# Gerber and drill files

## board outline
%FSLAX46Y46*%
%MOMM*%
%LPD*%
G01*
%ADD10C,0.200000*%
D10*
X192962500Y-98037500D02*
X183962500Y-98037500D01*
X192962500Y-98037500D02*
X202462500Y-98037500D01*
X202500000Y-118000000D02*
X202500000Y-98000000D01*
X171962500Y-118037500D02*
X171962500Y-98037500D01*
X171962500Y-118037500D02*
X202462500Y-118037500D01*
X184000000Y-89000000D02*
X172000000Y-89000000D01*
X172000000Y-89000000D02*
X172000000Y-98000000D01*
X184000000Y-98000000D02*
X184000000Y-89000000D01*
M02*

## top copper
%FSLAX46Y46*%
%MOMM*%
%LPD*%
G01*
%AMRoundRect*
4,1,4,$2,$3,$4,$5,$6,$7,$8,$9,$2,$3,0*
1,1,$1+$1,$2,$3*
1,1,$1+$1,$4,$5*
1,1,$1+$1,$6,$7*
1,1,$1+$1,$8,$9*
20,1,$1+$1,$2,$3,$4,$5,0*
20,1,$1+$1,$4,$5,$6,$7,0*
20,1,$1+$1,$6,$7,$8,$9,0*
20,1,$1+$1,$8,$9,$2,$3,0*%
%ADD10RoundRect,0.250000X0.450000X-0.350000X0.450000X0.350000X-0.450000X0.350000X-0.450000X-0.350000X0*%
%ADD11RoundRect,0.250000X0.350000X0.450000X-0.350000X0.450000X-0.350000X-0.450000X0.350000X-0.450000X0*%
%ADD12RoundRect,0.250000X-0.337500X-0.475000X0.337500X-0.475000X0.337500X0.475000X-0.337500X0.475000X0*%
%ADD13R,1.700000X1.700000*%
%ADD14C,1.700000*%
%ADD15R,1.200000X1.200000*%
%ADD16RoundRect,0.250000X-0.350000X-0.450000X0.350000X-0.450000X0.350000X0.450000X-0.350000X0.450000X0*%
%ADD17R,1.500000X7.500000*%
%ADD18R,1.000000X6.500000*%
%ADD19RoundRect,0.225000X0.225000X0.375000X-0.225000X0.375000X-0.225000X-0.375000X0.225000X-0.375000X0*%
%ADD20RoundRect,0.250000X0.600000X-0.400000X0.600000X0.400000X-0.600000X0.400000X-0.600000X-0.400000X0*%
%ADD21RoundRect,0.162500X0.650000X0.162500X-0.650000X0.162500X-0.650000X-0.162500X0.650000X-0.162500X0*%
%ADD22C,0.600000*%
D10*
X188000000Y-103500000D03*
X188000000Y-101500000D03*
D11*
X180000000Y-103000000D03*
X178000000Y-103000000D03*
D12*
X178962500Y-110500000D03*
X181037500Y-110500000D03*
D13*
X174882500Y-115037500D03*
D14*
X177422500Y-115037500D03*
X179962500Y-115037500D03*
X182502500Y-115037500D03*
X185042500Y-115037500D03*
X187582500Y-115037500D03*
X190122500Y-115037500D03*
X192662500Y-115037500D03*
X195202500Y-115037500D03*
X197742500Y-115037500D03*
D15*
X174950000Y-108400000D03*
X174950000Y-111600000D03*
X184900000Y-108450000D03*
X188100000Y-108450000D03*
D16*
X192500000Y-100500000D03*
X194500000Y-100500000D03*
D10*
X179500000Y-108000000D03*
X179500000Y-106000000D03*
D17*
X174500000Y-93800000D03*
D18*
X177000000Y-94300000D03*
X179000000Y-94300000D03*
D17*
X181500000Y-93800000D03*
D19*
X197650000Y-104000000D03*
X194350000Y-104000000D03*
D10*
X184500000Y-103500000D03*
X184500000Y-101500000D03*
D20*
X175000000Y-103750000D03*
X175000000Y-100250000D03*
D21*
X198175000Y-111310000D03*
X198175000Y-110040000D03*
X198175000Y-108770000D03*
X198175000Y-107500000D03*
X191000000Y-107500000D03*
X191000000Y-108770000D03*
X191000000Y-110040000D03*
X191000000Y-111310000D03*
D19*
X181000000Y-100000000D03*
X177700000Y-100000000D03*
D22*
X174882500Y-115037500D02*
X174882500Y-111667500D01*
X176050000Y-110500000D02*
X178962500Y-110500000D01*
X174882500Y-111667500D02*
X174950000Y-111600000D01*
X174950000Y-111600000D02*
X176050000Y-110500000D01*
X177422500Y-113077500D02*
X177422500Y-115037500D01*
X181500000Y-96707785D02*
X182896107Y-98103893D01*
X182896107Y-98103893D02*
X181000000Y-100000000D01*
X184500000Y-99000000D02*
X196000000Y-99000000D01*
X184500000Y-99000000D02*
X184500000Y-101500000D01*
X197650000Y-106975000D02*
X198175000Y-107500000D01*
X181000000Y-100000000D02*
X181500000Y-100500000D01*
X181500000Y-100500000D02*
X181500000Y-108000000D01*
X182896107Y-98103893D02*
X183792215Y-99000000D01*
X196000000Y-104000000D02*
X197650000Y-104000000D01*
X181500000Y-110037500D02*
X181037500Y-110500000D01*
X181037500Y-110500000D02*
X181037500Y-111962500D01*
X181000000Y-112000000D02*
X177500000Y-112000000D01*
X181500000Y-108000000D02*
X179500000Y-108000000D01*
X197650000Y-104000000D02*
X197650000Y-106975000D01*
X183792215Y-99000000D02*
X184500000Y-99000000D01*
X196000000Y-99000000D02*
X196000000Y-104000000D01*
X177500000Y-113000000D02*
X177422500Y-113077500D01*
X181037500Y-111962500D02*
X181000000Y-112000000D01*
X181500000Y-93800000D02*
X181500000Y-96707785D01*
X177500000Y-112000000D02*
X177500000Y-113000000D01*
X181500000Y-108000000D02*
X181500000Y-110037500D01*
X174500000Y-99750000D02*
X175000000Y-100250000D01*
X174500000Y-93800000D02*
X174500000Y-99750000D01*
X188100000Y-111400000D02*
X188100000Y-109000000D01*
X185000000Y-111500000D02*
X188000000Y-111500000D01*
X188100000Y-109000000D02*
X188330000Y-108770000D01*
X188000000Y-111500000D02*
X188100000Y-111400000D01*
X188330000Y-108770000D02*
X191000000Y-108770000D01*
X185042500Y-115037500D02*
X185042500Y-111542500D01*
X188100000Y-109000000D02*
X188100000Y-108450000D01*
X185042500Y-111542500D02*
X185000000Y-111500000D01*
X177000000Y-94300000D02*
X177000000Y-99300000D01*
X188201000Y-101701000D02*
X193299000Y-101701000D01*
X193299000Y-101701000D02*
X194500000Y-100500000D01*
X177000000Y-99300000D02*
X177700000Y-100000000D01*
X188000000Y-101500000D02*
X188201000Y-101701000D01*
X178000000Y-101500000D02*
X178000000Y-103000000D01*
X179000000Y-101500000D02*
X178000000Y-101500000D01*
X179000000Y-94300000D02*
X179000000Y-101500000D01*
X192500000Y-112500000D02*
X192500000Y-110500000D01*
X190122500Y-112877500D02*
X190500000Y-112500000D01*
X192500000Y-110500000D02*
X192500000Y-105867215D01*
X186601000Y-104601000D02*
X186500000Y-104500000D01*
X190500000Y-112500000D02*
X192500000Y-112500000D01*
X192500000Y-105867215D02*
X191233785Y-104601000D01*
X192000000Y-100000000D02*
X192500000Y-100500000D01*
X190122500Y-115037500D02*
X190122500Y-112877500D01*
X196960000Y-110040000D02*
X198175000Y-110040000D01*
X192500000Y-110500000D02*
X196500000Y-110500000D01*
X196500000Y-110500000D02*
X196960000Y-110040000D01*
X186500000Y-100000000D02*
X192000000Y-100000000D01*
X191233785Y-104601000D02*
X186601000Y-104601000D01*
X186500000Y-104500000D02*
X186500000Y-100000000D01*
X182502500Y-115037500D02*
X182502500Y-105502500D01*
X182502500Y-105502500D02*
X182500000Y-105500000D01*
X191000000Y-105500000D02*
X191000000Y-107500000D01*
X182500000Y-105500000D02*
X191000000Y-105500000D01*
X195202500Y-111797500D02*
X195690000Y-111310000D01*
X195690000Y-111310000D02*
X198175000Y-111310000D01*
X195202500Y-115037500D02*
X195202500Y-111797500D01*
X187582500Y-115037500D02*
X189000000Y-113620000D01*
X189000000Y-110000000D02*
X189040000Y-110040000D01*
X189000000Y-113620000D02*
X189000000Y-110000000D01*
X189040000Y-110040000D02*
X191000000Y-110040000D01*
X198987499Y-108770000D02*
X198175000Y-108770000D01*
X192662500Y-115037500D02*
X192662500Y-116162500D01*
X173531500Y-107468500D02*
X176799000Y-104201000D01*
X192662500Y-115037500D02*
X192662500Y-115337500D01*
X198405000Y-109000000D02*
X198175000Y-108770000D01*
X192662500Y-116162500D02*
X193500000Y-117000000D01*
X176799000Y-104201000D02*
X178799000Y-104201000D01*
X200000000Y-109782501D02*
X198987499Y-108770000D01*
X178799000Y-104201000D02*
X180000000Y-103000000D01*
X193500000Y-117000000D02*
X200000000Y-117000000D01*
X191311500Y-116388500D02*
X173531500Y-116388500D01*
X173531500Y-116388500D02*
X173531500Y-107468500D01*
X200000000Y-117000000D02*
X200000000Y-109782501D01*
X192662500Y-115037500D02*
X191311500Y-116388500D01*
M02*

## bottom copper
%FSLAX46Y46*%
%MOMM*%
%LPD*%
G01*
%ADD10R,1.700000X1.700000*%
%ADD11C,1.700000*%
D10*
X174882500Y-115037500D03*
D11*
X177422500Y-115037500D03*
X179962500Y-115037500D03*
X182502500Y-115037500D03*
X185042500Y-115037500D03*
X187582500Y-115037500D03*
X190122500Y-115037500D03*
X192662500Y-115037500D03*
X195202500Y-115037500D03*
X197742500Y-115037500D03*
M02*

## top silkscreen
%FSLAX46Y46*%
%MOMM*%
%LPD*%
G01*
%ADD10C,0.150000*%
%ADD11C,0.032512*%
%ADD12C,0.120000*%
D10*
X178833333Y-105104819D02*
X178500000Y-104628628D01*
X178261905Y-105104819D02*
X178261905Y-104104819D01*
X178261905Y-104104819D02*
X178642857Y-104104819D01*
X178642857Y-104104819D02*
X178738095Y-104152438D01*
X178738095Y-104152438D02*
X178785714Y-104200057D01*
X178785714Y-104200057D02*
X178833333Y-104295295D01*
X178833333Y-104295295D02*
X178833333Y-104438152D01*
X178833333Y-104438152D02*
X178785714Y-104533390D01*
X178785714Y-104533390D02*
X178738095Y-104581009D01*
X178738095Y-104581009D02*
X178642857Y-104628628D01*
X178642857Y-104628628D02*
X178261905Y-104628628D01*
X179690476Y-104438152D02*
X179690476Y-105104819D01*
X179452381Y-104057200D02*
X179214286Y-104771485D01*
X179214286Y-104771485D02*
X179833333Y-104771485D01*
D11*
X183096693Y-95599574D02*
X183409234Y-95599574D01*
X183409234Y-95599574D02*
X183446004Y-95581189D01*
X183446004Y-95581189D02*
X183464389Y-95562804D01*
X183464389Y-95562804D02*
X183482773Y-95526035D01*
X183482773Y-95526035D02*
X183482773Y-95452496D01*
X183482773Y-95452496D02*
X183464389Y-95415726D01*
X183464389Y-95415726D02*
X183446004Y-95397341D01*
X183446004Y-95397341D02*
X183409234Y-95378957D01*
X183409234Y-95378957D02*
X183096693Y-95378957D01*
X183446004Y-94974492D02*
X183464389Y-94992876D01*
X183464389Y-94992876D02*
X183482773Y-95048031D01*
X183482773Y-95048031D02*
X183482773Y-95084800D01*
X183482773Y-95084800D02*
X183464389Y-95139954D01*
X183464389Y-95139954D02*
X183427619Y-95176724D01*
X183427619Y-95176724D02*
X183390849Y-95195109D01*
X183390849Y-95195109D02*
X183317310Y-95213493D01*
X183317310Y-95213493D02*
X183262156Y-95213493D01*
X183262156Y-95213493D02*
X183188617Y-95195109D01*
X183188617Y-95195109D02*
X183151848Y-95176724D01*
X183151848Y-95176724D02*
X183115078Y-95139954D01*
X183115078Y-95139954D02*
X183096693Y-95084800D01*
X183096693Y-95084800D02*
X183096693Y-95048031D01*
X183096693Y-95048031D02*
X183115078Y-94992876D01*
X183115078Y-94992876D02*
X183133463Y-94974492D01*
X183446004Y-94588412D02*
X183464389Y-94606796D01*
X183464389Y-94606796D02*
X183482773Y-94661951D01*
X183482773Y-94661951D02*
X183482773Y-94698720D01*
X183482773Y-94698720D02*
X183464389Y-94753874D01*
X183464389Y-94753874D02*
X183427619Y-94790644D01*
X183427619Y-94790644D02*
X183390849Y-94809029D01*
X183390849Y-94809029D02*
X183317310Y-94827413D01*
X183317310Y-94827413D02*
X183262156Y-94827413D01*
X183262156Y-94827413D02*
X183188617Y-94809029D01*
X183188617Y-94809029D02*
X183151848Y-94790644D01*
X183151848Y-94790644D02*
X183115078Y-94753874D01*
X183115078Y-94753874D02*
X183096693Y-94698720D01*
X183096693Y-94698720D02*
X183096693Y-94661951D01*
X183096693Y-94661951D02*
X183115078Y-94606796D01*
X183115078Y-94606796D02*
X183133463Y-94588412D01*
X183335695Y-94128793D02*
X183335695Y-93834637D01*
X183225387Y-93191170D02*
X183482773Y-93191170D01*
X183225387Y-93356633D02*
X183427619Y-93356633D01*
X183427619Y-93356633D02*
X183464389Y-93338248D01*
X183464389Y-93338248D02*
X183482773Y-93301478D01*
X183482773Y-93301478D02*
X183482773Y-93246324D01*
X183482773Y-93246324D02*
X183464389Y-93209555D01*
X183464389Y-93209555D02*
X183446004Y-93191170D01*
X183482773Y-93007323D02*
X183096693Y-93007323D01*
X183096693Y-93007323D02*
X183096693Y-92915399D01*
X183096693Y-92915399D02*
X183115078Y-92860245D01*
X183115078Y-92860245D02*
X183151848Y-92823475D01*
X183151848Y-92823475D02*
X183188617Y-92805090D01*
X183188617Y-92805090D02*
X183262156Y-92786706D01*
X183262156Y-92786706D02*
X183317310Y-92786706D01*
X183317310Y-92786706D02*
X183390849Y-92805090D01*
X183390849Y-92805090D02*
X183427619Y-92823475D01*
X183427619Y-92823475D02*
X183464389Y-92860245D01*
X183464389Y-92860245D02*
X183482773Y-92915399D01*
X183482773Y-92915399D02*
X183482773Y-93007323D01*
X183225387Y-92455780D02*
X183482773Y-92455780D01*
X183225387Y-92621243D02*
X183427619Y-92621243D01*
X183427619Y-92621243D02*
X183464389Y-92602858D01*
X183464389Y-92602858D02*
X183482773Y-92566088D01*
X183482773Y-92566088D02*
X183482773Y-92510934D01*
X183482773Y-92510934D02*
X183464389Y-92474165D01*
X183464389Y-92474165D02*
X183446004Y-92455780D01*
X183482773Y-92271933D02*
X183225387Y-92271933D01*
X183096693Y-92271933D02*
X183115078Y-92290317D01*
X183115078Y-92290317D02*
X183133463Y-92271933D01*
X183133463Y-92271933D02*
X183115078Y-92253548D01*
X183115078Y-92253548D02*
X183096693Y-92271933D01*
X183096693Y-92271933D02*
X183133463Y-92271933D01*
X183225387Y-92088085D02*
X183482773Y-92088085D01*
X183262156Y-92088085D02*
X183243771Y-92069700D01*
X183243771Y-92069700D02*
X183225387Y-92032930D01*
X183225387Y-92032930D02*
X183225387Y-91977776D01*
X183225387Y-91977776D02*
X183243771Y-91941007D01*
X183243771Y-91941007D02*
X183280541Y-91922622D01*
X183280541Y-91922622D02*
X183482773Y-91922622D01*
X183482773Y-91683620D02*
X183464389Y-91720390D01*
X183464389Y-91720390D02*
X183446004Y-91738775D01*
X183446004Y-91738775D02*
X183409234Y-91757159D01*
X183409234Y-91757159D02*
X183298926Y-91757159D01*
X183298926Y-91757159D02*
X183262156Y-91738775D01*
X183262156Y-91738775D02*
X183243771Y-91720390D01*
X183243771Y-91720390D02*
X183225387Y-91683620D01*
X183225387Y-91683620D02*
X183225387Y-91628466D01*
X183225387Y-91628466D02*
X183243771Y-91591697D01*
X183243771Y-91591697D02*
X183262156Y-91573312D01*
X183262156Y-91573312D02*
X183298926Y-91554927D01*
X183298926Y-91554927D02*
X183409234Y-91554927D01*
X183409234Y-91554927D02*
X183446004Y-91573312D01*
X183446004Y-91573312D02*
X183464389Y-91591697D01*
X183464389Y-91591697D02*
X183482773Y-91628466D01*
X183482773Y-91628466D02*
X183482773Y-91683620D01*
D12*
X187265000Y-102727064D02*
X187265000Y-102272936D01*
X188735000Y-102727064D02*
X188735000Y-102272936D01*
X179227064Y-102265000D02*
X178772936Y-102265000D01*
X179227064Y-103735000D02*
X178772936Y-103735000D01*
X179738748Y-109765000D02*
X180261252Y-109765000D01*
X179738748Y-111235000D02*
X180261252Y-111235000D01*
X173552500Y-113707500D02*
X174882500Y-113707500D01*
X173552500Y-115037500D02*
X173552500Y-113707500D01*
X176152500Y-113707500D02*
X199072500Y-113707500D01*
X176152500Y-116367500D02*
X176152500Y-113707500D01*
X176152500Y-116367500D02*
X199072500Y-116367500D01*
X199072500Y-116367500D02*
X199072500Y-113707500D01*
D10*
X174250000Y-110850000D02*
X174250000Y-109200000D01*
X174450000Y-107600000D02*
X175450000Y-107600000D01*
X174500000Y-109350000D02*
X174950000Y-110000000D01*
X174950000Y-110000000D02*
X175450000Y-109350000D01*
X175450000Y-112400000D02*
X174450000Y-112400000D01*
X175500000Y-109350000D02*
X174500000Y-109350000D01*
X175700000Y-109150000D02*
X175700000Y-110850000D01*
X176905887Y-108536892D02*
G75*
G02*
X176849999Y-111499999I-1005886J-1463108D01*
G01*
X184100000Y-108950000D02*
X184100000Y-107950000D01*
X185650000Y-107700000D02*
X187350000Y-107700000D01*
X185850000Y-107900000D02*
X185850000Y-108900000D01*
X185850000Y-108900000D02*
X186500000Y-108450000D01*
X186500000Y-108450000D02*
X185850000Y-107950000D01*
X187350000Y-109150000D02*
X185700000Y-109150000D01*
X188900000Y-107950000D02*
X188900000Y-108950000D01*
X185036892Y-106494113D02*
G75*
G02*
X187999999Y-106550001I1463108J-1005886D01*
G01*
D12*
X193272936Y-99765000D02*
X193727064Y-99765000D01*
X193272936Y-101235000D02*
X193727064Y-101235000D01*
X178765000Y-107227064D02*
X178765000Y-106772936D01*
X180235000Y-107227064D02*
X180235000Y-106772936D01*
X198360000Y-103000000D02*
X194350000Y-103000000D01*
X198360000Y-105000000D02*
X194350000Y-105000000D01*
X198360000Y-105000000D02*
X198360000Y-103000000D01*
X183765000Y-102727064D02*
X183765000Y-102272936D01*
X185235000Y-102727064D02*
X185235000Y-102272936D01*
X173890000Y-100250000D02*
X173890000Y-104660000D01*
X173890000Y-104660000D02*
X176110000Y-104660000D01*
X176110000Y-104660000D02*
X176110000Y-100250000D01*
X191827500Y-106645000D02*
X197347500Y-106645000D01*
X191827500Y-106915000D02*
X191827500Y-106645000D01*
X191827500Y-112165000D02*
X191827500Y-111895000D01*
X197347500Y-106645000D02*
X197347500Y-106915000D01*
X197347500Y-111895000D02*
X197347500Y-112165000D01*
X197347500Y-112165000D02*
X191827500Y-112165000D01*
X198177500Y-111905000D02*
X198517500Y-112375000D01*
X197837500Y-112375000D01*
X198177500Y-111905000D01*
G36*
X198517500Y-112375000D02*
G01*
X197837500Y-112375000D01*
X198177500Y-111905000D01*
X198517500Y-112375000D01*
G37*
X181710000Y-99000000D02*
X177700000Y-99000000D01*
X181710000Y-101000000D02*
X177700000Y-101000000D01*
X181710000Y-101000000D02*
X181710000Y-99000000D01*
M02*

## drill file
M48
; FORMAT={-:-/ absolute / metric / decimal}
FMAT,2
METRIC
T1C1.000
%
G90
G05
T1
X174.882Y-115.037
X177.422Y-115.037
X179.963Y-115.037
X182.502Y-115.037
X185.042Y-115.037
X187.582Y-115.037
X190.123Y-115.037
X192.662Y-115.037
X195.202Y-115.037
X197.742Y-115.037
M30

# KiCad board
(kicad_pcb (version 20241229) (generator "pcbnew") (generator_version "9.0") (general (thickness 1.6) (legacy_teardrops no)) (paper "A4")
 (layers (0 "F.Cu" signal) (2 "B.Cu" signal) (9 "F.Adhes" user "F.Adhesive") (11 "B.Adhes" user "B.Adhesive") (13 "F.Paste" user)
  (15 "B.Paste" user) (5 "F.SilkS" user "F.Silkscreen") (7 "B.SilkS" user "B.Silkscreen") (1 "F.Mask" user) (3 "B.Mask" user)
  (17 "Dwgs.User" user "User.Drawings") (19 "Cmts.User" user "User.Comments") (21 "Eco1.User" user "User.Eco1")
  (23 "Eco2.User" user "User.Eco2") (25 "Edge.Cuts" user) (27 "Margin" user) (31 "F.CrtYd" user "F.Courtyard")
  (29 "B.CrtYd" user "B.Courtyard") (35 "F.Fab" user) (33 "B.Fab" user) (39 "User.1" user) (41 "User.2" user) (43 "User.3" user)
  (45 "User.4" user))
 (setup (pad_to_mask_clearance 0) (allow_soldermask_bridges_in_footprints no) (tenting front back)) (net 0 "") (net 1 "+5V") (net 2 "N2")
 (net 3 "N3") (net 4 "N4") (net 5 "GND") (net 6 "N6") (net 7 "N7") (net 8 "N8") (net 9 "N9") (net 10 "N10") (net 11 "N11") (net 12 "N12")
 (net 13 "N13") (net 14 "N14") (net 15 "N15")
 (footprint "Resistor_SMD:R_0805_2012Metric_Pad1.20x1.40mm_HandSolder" (layer "F.Cu") (at 188 102.5 90)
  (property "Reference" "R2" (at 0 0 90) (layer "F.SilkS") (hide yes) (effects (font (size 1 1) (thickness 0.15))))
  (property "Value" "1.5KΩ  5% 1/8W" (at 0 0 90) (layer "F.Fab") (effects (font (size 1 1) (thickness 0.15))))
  (fp_line (start -0.227064 -0.735) (end 0.227064 -0.735) (stroke (width 0.12) (type solid)) (layer "F.SilkS"))
  (fp_line (start -0.227064 0.735) (end 0.227064 0.735) (stroke (width 0.12) (type solid)) (layer "F.SilkS"))
  (pad "1" smd roundrect (at -1 0 90) (size 1.2 1.4) (layers "F.Cu" "F.Mask" "F.Paste") (roundrect_rratio 0.208333) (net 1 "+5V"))
  (pad "2" smd roundrect (at 1 0 90) (size 1.2 1.4) (layers "F.Cu" "F.Mask" "F.Paste") (roundrect_rratio 0.208333) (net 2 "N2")))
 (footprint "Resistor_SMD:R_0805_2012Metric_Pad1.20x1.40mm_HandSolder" (layer "F.Cu") (at 179 103 180)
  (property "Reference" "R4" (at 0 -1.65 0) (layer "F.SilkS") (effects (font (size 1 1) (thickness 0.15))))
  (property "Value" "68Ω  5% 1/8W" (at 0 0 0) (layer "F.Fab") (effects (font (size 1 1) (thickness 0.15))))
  (fp_line (start -0.227064 0.735) (end 0.227064 0.735) (stroke (width 0.12) (type solid)) (layer "F.SilkS"))
  (fp_line (start -0.227064 -0.735) (end 0.227064 -0.735) (stroke (width 0.12) (type solid)) (layer "F.SilkS"))
  (pad "1" smd roundrect (at -1 0 180) (size 1.2 1.4) (layers "F.Cu" "F.Mask" "F.Paste") (roundrect_rratio 0.208333) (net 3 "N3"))
  (pad "2" smd roundrect (at 1 0 180) (size 1.2 1.4) (layers "F.Cu" "F.Mask" "F.Paste") (roundrect_rratio 0.208333) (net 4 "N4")))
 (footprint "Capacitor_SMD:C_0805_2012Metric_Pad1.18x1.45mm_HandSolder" (layer "F.Cu") (at 180 110.5)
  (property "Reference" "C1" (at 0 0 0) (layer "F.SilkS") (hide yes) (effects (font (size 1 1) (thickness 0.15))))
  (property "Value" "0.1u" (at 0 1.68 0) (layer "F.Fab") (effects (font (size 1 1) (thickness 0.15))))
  (fp_line (start -0.261252 -0.735) (end 0.261252 -0.735) (stroke (width 0.12) (type solid)) (layer "F.SilkS"))
  (fp_line (start -0.261252 0.735) (end 0.261252 0.735) (stroke (width 0.12) (type solid)) (layer "F.SilkS"))
  (pad "1" smd roundrect (at -1.0375 0) (size 1.175 1.45) (layers "F.Cu" "F.Mask" "F.Paste") (roundrect_rratio 0.212766) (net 1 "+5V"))
  (pad "2" smd roundrect (at 1.0375 0) (size 1.175 1.45) (layers "F.Cu" "F.Mask" "F.Paste") (roundrect_rratio 0.212766) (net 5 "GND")))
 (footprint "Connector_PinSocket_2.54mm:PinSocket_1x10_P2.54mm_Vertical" (layer "F.Cu") (at 174.8825 115.0375 90)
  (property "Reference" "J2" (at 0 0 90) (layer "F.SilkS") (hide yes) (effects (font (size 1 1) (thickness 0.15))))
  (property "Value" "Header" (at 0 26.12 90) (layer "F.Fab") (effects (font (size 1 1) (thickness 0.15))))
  (fp_line (start 1.33 -1.33) (end 1.33 0) (stroke (width 0.12) (type solid)) (layer "F.SilkS"))
  (fp_line (start 0 -1.33) (end 1.33 -1.33) (stroke (width 0.12) (type solid)) (layer "F.SilkS"))
  (fp_line (start 1.33 1.27) (end 1.33 24.19) (stroke (width 0.12) (type solid)) (layer "F.SilkS"))
  (fp_line (start -1.33 1.27) (end 1.33 1.27) (stroke (width 0.12) (type solid)) (layer "F.SilkS"))
  (fp_line (start -1.33 1.27) (end -1.33 24.19) (stroke (width 0.12) (type solid)) (layer "F.SilkS"))
  (fp_line (start -1.33 24.19) (end 1.33 24.19) (stroke (width 0.12) (type solid)) (layer "F.SilkS"))
  (pad "1" thru_hole rect (at 0 0 90) (size 1.7 1.7) (drill 1) (layers "*.Cu" "*.Mask") (remove_unused_layers no) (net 1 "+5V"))
  (pad "2" thru_hole circle (at 0 2.54 90) (size 1.7 1.7) (drill 1) (layers "*.Cu" "*.Mask") (remove_unused_layers no) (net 5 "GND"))
  (pad "3" thru_hole circle (at 0 5.08 90) (size 1.7 1.7) (drill 1) (layers "*.Cu" "*.Mask") (remove_unused_layers no) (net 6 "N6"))
  (pad "4" thru_hole circle (at 0 7.62 90) (size 1.7 1.7) (drill 1) (layers "*.Cu" "*.Mask") (remove_unused_layers no) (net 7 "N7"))
  (pad "5" thru_hole circle (at 0 10.16 90) (size 1.7 1.7) (drill 1) (layers "*.Cu" "*.Mask") (remove_unused_layers no) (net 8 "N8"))
  (pad "6" thru_hole circle (at 0 12.7 90) (size 1.7 1.7) (drill 1) (layers "*.Cu" "*.Mask") (remove_unused_layers no) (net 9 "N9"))
  (pad "7" thru_hole circle (at 0 15.24 90) (size 1.7 1.7) (drill 1) (layers "*.Cu" "*.Mask") (remove_unused_layers no) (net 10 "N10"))
  (pad "8" thru_hole circle (at 0 17.78 90) (size 1.7 1.7) (drill 1) (layers "*.Cu" "*.Mask") (remove_unused_layers no) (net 3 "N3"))
  (pad "9" thru_hole circle (at 0 20.32 90) (size 1.7 1.7) (drill 1) (layers "*.Cu" "*.Mask") (remove_unused_layers no) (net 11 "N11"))
  (pad "10" thru_hole circle (at 0 22.86 90) (size 1.7 1.7) (drill 1) (layers "*.Cu" "*.Mask") (remove_unused_layers no) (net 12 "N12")))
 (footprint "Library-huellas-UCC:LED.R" (layer "F.Cu") (at 175.4 110.5 -90)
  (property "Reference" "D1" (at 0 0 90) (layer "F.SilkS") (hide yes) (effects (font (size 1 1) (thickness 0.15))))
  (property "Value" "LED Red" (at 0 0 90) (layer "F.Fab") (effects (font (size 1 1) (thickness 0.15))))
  (fp_line (start 0.35 1.15) (end -1.3 1.15) (stroke (width 0.15) (type solid)) (layer "F.SilkS"))
  (fp_line (start -2.9 0.95) (end -2.9 -0.05) (stroke (width 0.15) (type solid)) (layer "F.SilkS"))
  (fp_line (start -1.15 0.9) (end -0.5 0.45) (stroke (width 0.15) (type solid)) (layer "F.SilkS"))
  (fp_line (start -0.5 0.45) (end -1.15 -0.05) (stroke (width 0.15) (type solid)) (layer "F.SilkS"))
  (fp_line (start 1.9 -0.05) (end 1.9 0.95) (stroke (width 0.15) (type solid)) (layer "F.SilkS"))
  (fp_line (start -1.15 -0.1) (end -1.15 0.9) (stroke (width 0.15) (type solid)) (layer "F.SilkS"))
  (fp_line (start -1.35 -0.3) (end 0.35 -0.3) (stroke (width 0.15) (type solid)) (layer "F.SilkS"))
  (fp_arc (start -1.963108 -1.505887) (mid -0.466517 -2.275211) (end 0.999999 -1.449999) (stroke (width 0.15) (type solid))
   (layer "F.SilkS"))
  (pad "1" smd rect (at -2.1 0.45 270) (size 1.2 1.2) (layers "F.Cu" "F.Mask" "F.Paste") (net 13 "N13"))
  (pad "2" smd rect (at 1.1 0.45 270) (size 1.2 1.2) (layers "F.Cu" "F.Mask" "F.Paste") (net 1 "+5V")))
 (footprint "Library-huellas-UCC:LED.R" (layer "F.Cu") (at 187 108)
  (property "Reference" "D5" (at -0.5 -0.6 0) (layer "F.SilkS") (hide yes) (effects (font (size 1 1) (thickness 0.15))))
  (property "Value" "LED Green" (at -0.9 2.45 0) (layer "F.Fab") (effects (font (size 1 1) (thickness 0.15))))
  (fp_line (start -2.9 0.95) (end -2.9 -0.05) (stroke (width 0.15) (type solid)) (layer "F.SilkS"))
  (fp_line (start -1.35 -0.3) (end 0.35 -0.3) (stroke (width 0.15) (type solid)) (layer "F.SilkS"))
  (fp_line (start -1.15 -0.1) (end -1.15 0.9) (stroke (width 0.15) (type solid)) (layer "F.SilkS"))
  (fp_line (start -1.15 0.9) (end -0.5 0.45) (stroke (width 0.15) (type solid)) (layer "F.SilkS"))
  (fp_line (start -0.5 0.45) (end -1.15 -0.05) (stroke (width 0.15) (type solid)) (layer "F.SilkS"))
  (fp_line (start 0.35 1.15) (end -1.3 1.15) (stroke (width 0.15) (type solid)) (layer "F.SilkS"))
  (fp_line (start 1.9 -0.05) (end 1.9 0.95) (stroke (width 0.15) (type solid)) (layer "F.SilkS"))
  (fp_arc (start -1.963108 -1.505887) (mid -0.466517 -2.275211) (end 0.999999 -1.449999) (stroke (width 0.15) (type solid))
   (layer "F.SilkS"))
  (pad "1" smd rect (at -2.1 0.45) (size 1.2 1.2) (layers "F.Cu" "F.Mask" "F.Paste") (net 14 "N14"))
  (pad "2" smd rect (at 1.1 0.45) (size 1.2 1.2) (layers "F.Cu" "F.Mask" "F.Paste") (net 8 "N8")))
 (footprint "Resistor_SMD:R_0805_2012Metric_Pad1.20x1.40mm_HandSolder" (layer "F.Cu") (at 193.5 100.5)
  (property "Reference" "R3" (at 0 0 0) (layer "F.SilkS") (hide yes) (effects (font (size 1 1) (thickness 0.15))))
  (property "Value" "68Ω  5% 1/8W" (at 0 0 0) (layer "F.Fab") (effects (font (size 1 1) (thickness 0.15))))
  (fp_line (start -0.227064 -0.735) (end 0.227064 -0.735) (stroke (width 0.12) (type solid)) (layer "F.SilkS"))
  (fp_line (start -0.227064 0.735) (end 0.227064 0.735) (stroke (width 0.12) (type solid)) (layer "F.SilkS"))
  (pad "1" smd roundrect (at -1 0) (size 1.2 1.4) (layers "F.Cu" "F.Mask" "F.Paste") (roundrect_rratio 0.208333) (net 10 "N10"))
  (pad "2" smd roundrect (at 1 0) (size 1.2 1.4) (layers "F.Cu" "F.Mask" "F.Paste") (roundrect_rratio 0.208333) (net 2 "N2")))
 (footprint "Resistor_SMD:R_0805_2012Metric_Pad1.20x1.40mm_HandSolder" (layer "F.Cu") (at 179.5 107 90)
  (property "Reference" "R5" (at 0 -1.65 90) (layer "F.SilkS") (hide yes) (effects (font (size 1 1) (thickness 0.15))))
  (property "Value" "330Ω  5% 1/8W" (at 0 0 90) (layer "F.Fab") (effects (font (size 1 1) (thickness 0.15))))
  (fp_line (start -0.227064 -0.735) (end 0.227064 -0.735) (stroke (width 0.12) (type solid)) (layer "F.SilkS"))
  (fp_line (start -0.227064 0.735) (end 0.227064 0.735) (stroke (width 0.12) (type solid)) (layer "F.SilkS"))
  (pad "1" smd roundrect (at -1 0 90) (size 1.2 1.4) (layers "F.Cu" "F.Mask" "F.Paste") (roundrect_rratio 0.208333) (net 5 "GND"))
  (pad "2" smd roundrect (at 1 0 90) (size 1.2 1.4) (layers "F.Cu" "F.Mask" "F.Paste") (roundrect_rratio 0.208333) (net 14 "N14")))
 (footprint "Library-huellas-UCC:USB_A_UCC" (layer "F.Cu") (at 178 94 -90)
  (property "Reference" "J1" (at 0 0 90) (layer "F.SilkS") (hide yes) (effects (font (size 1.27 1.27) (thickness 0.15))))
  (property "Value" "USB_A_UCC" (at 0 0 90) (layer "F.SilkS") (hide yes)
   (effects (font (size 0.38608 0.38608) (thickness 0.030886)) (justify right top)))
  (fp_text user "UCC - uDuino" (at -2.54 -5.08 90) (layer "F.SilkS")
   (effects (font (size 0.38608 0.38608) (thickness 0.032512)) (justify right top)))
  (pad "1" smd rect (at -0.2 3.5 270) (size 7.5 1.5) (layers "F.Cu" "F.Mask" "F.Paste") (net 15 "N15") (solder_mask_margin 0.1016))
  (pad "2" smd rect (at 0.3 1 270) (size 6.5 1) (layers "F.Cu" "F.Mask" "F.Paste") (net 2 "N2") (solder_mask_margin 0.1016))
  (pad "3" smd rect (at 0.3 -1 270) (size 6.5 1) (layers "F.Cu" "F.Mask" "F.Paste") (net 4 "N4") (solder_mask_margin 0.1016))
  (pad "4" smd rect (at -0.2 -3.5 270) (size 7.5 1.5) (layers "F.Cu" "F.Mask" "F.Paste") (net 5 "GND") (solder_mask_margin 0.1016)))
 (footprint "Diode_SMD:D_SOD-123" (layer "F.Cu") (at 196 104 180)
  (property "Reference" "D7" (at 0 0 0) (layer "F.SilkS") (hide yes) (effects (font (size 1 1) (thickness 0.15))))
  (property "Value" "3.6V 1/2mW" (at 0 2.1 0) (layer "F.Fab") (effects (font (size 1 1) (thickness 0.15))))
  (fp_line (start -2.36 1) (end 1.65 1) (stroke (width 0.12) (type solid)) (layer "F.SilkS"))
  (fp_line (start -2.36 -1) (end 1.65 -1) (stroke (width 0.12) (type solid)) (layer "F.SilkS"))
  (fp_line (start -2.36 -1) (end -2.36 1) (stroke (width 0.12) (type solid)) (layer "F.SilkS"))
  (pad "1" smd roundrect (at -1.65 0 180) (size 0.9 1.2) (layers "F.Cu" "F.Mask" "F.Paste") (roundrect_rratio 0.25) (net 5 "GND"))
  (pad "2" smd roundrect (at 1.65 0 180) (size 0.9 1.2) (layers "F.Cu" "F.Mask" "F.Paste") (roundrect_rratio 0.25) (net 4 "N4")))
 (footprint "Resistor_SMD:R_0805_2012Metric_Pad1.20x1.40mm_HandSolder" (layer "F.Cu") (at 184.5 102.5 90)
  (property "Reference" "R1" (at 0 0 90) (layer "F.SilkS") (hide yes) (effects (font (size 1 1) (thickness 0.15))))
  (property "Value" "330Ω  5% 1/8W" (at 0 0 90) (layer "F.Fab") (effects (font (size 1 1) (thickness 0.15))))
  (fp_line (start -0.227064 -0.735) (end 0.227064 -0.735) (stroke (width 0.12) (type solid)) (layer "F.SilkS"))
  (fp_line (start -0.227064 0.735) (end 0.227064 0.735) (stroke (width 0.12) (type solid)) (layer "F.SilkS"))
  (pad "1" smd roundrect (at -1 0 90) (size 1.2 1.4) (layers "F.Cu" "F.Mask" "F.Paste") (roundrect_rratio 0.208333) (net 13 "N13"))
  (pad "2" smd roundrect (at 1 0 90) (size 1.2 1.4) (layers "F.Cu" "F.Mask" "F.Paste") (roundrect_rratio 0.208333) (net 5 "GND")))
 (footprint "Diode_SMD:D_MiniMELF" (layer "F.Cu") (at 175 102 90)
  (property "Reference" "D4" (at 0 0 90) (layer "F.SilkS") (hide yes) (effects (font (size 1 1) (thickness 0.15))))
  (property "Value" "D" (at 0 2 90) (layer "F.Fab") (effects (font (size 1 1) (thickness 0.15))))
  (fp_line (start 1.75 -1.11) (end -2.66 -1.11) (stroke (width 0.12) (type solid)) (layer "F.SilkS"))
  (fp_line (start -2.66 -1.11) (end -2.66 1.11) (stroke (width 0.12) (type solid)) (layer "F.SilkS"))
  (fp_line (start -2.66 1.11) (end 1.75 1.11) (stroke (width 0.12) (type solid)) (layer "F.SilkS"))
  (pad "1" smd roundrect (at -1.75 0 90) (size 1.3 1.7) (layers "F.Cu" "F.Mask" "F.Paste") (roundrect_rratio 0.1923076923) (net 1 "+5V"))
  (pad "2" smd roundrect (at 1.75 0 90) (size 1.3 1.7) (layers "F.Cu" "F.Mask" "F.Paste") (roundrect_rratio 0.1923076923) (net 15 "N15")))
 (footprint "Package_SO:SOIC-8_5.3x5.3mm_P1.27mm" (layer "F.Cu") (at 194.5875 109.405 180)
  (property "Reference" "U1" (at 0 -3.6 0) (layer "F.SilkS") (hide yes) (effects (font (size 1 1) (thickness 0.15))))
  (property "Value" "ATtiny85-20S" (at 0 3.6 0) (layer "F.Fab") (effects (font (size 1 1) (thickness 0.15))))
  (fp_line (start 2.76 2.76) (end -2.76 2.76) (stroke (width 0.12) (type solid)) (layer "F.SilkS"))
  (fp_line (start 2.76 2.49) (end 2.76 2.76) (stroke (width 0.12) (type solid)) (layer "F.SilkS"))
  (fp_line (start 2.76 -2.76) (end 2.76 -2.49) (stroke (width 0.12) (type solid)) (layer "F.SilkS"))
  (fp_line (start -2.76 2.76) (end -2.76 2.49) (stroke (width 0.12) (type solid)) (layer "F.SilkS"))
  (fp_line (start -2.76 -2.49) (end -2.76 -2.76) (stroke (width 0.12) (type solid)) (layer "F.SilkS"))
  (fp_line (start -2.76 -2.76) (end 2.76 -2.76) (stroke (width 0.12) (type solid)) (layer "F.SilkS"))
  (fp_poly (pts (xy -3.59 -2.5) (xy -3.93 -2.97) (xy -3.25 -2.97)) (stroke (width 0.12) (type solid)) (fill yes) (layer "F.SilkS"))
  (pad "1" smd roundrect (at -3.5875 -1.905 180) (size 1.625 0.65) (layers "F.Cu" "F.Mask" "F.Paste") (roundrect_rratio 0.25) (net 11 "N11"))
  (pad "2" smd roundrect (at -3.5875 -0.635 180) (size 1.625 0.65) (layers "F.Cu" "F.Mask" "F.Paste") (roundrect_rratio 0.25) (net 10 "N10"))
  (pad "3" smd roundrect (at -3.5875 0.635 180) (size 1.625 0.65) (layers "F.Cu" "F.Mask" "F.Paste") (roundrect_rratio 0.25) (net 3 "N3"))
  (pad "4" smd roundrect (at -3.5875 1.905 180) (size 1.625 0.65) (layers "F.Cu" "F.Mask" "F.Paste") (roundrect_rratio 0.25) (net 5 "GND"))
  (pad "5" smd roundrect (at 3.5875 1.905 180) (size 1.625 0.65) (layers "F.Cu" "F.Mask" "F.Paste") (roundrect_rratio 0.25) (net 7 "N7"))
  (pad "6" smd roundrect (at 3.5875 0.635 180) (size 1.625 0.65) (layers "F.Cu" "F.Mask" "F.Paste") (roundrect_rratio 0.25) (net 8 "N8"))
  (pad "7" smd roundrect (at 3.5875 -0.635 180) (size 1.625 0.65) (layers "F.Cu" "F.Mask" "F.Paste") (roundrect_rratio 0.25) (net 9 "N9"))
  (pad "8" smd roundrect (at 3.5875 -1.905 180) (size 1.625 0.65) (layers "F.Cu" "F.Mask" "F.Paste") (roundrect_rratio 0.25) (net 1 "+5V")))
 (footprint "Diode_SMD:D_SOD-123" (layer "F.Cu") (at 179.35 100 180)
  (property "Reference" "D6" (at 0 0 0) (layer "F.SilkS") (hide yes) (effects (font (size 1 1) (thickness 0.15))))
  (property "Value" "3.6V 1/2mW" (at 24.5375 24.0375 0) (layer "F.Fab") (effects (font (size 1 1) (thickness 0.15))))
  (fp_line (start -2.36 1) (end 1.65 1) (stroke (width 0.12) (type solid)) (layer "F.SilkS"))
  (fp_line (start -2.36 -1) (end 1.65 -1) (stroke (width 0.12) (type solid)) (layer "F.SilkS"))
  (fp_line (start -2.36 -1) (end -2.36 1) (stroke (width 0.12) (type solid)) (layer "F.SilkS"))
  (pad "1" smd roundrect (at -1.65 0 180) (size 0.9 1.2) (layers "F.Cu" "F.Mask" "F.Paste") (roundrect_rratio 0.25) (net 5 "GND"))
  (pad "2" smd roundrect (at 1.65 0 180) (size 0.9 1.2) (layers "F.Cu" "F.Mask" "F.Paste") (roundrect_rratio 0.25) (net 2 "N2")))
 (gr_line (start 192.9625 98.0375) (end 183.9625 98.0375) (stroke (width 0.2) (type solid)) (layer "Edge.Cuts"))
 (gr_line (start 192.9625 98.0375) (end 202.4625 98.0375) (stroke (width 0.2) (type solid)) (layer "Edge.Cuts"))
 (gr_line (start 202.5 118) (end 202.5 98) (stroke (width 0.2) (type solid)) (layer "Edge.Cuts"))
 (gr_line (start 171.9625 118.0375) (end 171.9625 98.0375) (stroke (width 0.2) (type solid)) (layer "Edge.Cuts"))
 (gr_line (start 171.9625 118.0375) (end 202.4625 118.0375) (stroke (width 0.2) (type solid)) (layer "Edge.Cuts"))
 (gr_line (start 184 89) (end 172 89) (stroke (width 0.2) (type solid)) (layer "Edge.Cuts"))
 (gr_line (start 172 89) (end 172 98) (stroke (width 0.2) (type solid)) (layer "Edge.Cuts"))
 (gr_line (start 184 98) (end 184 89) (stroke (width 0.2) (type solid)) (layer "Edge.Cuts"))
 (segment (start 174.8825 115.0375) (end 174.8825 111.6675) (width 0.6) (layer "F.Cu") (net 1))
 (segment (start 176.05 110.5) (end 178.9625 110.5) (width 0.6) (layer "F.Cu") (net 1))
 (segment (start 174.8825 111.6675) (end 174.95 111.6) (width 0.6) (layer "F.Cu") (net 1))
 (segment (start 174.95 111.6) (end 176.05 110.5) (width 0.6) (layer "F.Cu") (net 1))
 (segment (start 177.4225 113.0775) (end 177.4225 115.0375) (width 0.6) (layer "F.Cu") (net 5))
 (segment (start 181.5 96.707785) (end 182.896107 98.103893) (width 0.6) (layer "F.Cu") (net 5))
 (segment (start 182.896107 98.103893) (end 181 100) (width 0.6) (layer "F.Cu") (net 5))
 (segment (start 184.5 99) (end 196 99) (width 0.6) (layer "F.Cu") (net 5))
 (segment (start 184.5 99) (end 184.5 101.5) (width 0.6) (layer "F.Cu") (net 5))
 (segment (start 197.65 106.975) (end 198.175 107.5) (width 0.6) (layer "F.Cu") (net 5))
 (segment (start 181 100) (end 181.5 100.5) (width 0.6) (layer "F.Cu") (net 5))
 (segment (start 181.5 100.5) (end 181.5 108) (width 0.6) (layer "F.Cu") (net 5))
 (segment (start 182.896107 98.103893) (end 183.792215 99) (width 0.6) (layer "F.Cu") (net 5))
 (segment (start 196 104) (end 197.65 104) (width 0.6) (layer "F.Cu") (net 5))
 (segment (start 181.5 110.0375) (end 181.0375 110.5) (width 0.6) (layer "F.Cu") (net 5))
 (segment (start 181.0375 110.5) (end 181.0375 111.9625) (width 0.6) (layer "F.Cu") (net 5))
 (segment (start 181 112) (end 177.5 112) (width 0.6) (layer "F.Cu") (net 5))
 (segment (start 181.5 108) (end 179.5 108) (width 0.6) (layer "F.Cu") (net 5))
 (segment (start 197.65 104) (end 197.65 106.975) (width 0.6) (layer "F.Cu") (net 5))
 (segment (start 183.792215 99) (end 184.5 99) (width 0.6) (layer "F.Cu") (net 5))
 (segment (start 196 99) (end 196 104) (width 0.6) (layer "F.Cu") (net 5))
 (segment (start 177.5 113) (end 177.4225 113.0775) (width 0.6) (layer "F.Cu") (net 5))
 (segment (start 181.0375 111.9625) (end 181 112) (width 0.6) (layer "F.Cu") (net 5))
 (segment (start 181.5 93.8) (end 181.5 96.707785) (width 0.6) (layer "F.Cu") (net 5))
 (segment (start 177.5 112) (end 177.5 113) (width 0.6) (layer "F.Cu") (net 5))
 (segment (start 181.5 108) (end 181.5 110.0375) (width 0.6) (layer "F.Cu") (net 5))
 (segment (start 174.5 99.75) (end 175 100.25) (width 0.6) (layer "F.Cu") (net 15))
 (segment (start 174.5 93.8) (end 174.5 99.75) (width 0.6) (layer "F.Cu") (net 15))
 (segment (start 188.1 111.4) (end 188.1 109) (width 0.6) (layer "F.Cu") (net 8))
 (segment (start 185 111.5) (end 188 111.5) (width 0.6) (layer "F.Cu") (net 8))
 (segment (start 188.1 109) (end 188.33 108.77) (width 0.6) (layer "F.Cu") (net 8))
 (segment (start 188 111.5) (end 188.1 111.4) (width 0.6) (layer "F.Cu") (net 8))
 (segment (start 188.33 108.77) (end 191 108.77) (width 0.6) (layer "F.Cu") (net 8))
 (segment (start 185.0425 115.0375) (end 185.0425 111.5425) (width 0.6) (layer "F.Cu") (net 8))
 (segment (start 188.1 109) (end 188.1 108.45) (width 0.6) (layer "F.Cu") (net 8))
 (segment (start 185.0425 111.5425) (end 185 111.5) (width 0.6) (layer "F.Cu") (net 8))
 (segment (start 177 94.3) (end 177 99.3) (width 0.6) (layer "F.Cu") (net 2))
 (segment (start 188.201 101.701) (end 193.299 101.701) (width 0.6) (layer "F.Cu") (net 2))
 (segment (start 193.299 101.701) (end 194.5 100.5) (width 0.6) (layer "F.Cu") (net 2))
 (segment (start 177 99.3) (end 177.7 100) (width 0.6) (layer "F.Cu") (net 2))
 (segment (start 188 101.5) (end 188.201 101.701) (width 0.6) (layer "F.Cu") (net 2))
 (segment (start 178 101.5) (end 178 103) (width 0.6) (layer "F.Cu") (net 4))
 (segment (start 179 101.5) (end 178 101.5) (width 0.6) (layer "F.Cu") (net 4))
 (segment (start 179 94.3) (end 179 101.5) (width 0.6) (layer "F.Cu") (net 4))
 (segment (start 192.5 112.5) (end 192.5 110.5) (width 0.6) (layer "F.Cu") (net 10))
 (segment (start 190.1225 112.8775) (end 190.5 112.5) (width 0.6) (layer "F.Cu") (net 10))
 (segment (start 192.5 110.5) (end 192.5 105.867215) (width 0.6) (layer "F.Cu") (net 10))
 (segment (start 186.601 104.601) (end 186.5 104.5) (width 0.6) (layer "F.Cu") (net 10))
 (segment (start 190.5 112.5) (end 192.5 112.5) (width 0.6) (layer "F.Cu") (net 10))
 (segment (start 192.5 105.867215) (end 191.233785 104.601) (width 0.6) (layer "F.Cu") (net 10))
 (segment (start 192 100) (end 192.5 100.5) (width 0.6) (layer "F.Cu") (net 10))
 (segment (start 190.1225 115.0375) (end 190.1225 112.8775) (width 0.6) (layer "F.Cu") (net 10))
 (segment (start 196.96 110.04) (end 198.175 110.04) (width 0.6) (layer "F.Cu") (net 10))
 (segment (start 192.5 110.5) (end 196.5 110.5) (width 0.6) (layer "F.Cu") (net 10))
 (segment (start 196.5 110.5) (end 196.96 110.04) (width 0.6) (layer "F.Cu") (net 10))
 (segment (start 186.5 100) (end 192 100) (width 0.6) (layer "F.Cu") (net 10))
 (segment (start 191.233785 104.601) (end 186.601 104.601) (width 0.6) (layer "F.Cu") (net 10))
 (segment (start 186.5 104.5) (end 186.5 100) (width 0.6) (layer "F.Cu") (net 10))
 (segment (start 182.5025 115.0375) (end 182.5025 105.5025) (width 0.6) (layer "F.Cu") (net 7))
 (segment (start 182.5025 105.5025) (end 182.5 105.5) (width 0.6) (layer "F.Cu") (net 7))
 (segment (start 191 105.5) (end 191 107.5) (width 0.6) (layer "F.Cu") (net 7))
 (segment (start 182.5 105.5) (end 191 105.5) (width 0.6) (layer "F.Cu") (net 7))
 (segment (start 195.2025 111.7975) (end 195.69 111.31) (width 0.6) (layer "F.Cu") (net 11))
 (segment (start 195.69 111.31) (end 198.175 111.31) (width 0.6) (layer "F.Cu") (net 11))
 (segment (start 195.2025 115.0375) (end 195.2025 111.7975) (width 0.6) (layer "F.Cu") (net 11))
 (segment (start 187.5825 115.0375) (end 189 113.62) (width 0.6) (layer "F.Cu") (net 9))
 (segment (start 189 110) (end 189.04 110.04) (width 0.6) (layer "F.Cu") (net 9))
 (segment (start 189 113.62) (end 189 110) (width 0.6) (layer "F.Cu") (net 9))
 (segment (start 189.04 110.04) (end 191 110.04) (width 0.6) (layer "F.Cu") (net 9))
 (segment (start 198.987499 108.77) (end 198.175 108.77) (width 0.6) (layer "F.Cu") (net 3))
 (segment (start 192.6625 115.0375) (end 192.6625 116.1625) (width 0.6) (layer "F.Cu") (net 3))
 (segment (start 173.5315 107.4685) (end 176.799 104.201) (width 0.6) (layer "F.Cu") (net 3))
 (segment (start 192.6625 115.0375) (end 192.6625 115.3375) (width 0.6) (layer "F.Cu") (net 3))
 (segment (start 198.405 109) (end 198.175 108.77) (width 0.6) (layer "F.Cu") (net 3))
 (segment (start 192.6625 116.1625) (end 193.5 117) (width 0.6) (layer "F.Cu") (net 3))
 (segment (start 176.799 104.201) (end 178.799 104.201) (width 0.6) (layer "F.Cu") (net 3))
 (segment (start 200 109.782501) (end 198.987499 108.77) (width 0.6) (layer "F.Cu") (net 3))
 (segment (start 178.799 104.201) (end 180 103) (width 0.6) (layer "F.Cu") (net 3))
 (segment (start 193.5 117) (end 200 117) (width 0.6) (layer "F.Cu") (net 3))
 (segment (start 191.3115 116.3885) (end 173.5315 116.3885) (width 0.6) (layer "F.Cu") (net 3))
 (segment (start 173.5315 116.3885) (end 173.5315 107.4685) (width 0.6) (layer "F.Cu") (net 3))
 (segment (start 200 117) (end 200 109.782501) (width 0.6) (layer "F.Cu") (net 3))
 (segment (start 192.6625 115.0375) (end 191.3115 116.3885) (width 0.6) (layer "F.Cu") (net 3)))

